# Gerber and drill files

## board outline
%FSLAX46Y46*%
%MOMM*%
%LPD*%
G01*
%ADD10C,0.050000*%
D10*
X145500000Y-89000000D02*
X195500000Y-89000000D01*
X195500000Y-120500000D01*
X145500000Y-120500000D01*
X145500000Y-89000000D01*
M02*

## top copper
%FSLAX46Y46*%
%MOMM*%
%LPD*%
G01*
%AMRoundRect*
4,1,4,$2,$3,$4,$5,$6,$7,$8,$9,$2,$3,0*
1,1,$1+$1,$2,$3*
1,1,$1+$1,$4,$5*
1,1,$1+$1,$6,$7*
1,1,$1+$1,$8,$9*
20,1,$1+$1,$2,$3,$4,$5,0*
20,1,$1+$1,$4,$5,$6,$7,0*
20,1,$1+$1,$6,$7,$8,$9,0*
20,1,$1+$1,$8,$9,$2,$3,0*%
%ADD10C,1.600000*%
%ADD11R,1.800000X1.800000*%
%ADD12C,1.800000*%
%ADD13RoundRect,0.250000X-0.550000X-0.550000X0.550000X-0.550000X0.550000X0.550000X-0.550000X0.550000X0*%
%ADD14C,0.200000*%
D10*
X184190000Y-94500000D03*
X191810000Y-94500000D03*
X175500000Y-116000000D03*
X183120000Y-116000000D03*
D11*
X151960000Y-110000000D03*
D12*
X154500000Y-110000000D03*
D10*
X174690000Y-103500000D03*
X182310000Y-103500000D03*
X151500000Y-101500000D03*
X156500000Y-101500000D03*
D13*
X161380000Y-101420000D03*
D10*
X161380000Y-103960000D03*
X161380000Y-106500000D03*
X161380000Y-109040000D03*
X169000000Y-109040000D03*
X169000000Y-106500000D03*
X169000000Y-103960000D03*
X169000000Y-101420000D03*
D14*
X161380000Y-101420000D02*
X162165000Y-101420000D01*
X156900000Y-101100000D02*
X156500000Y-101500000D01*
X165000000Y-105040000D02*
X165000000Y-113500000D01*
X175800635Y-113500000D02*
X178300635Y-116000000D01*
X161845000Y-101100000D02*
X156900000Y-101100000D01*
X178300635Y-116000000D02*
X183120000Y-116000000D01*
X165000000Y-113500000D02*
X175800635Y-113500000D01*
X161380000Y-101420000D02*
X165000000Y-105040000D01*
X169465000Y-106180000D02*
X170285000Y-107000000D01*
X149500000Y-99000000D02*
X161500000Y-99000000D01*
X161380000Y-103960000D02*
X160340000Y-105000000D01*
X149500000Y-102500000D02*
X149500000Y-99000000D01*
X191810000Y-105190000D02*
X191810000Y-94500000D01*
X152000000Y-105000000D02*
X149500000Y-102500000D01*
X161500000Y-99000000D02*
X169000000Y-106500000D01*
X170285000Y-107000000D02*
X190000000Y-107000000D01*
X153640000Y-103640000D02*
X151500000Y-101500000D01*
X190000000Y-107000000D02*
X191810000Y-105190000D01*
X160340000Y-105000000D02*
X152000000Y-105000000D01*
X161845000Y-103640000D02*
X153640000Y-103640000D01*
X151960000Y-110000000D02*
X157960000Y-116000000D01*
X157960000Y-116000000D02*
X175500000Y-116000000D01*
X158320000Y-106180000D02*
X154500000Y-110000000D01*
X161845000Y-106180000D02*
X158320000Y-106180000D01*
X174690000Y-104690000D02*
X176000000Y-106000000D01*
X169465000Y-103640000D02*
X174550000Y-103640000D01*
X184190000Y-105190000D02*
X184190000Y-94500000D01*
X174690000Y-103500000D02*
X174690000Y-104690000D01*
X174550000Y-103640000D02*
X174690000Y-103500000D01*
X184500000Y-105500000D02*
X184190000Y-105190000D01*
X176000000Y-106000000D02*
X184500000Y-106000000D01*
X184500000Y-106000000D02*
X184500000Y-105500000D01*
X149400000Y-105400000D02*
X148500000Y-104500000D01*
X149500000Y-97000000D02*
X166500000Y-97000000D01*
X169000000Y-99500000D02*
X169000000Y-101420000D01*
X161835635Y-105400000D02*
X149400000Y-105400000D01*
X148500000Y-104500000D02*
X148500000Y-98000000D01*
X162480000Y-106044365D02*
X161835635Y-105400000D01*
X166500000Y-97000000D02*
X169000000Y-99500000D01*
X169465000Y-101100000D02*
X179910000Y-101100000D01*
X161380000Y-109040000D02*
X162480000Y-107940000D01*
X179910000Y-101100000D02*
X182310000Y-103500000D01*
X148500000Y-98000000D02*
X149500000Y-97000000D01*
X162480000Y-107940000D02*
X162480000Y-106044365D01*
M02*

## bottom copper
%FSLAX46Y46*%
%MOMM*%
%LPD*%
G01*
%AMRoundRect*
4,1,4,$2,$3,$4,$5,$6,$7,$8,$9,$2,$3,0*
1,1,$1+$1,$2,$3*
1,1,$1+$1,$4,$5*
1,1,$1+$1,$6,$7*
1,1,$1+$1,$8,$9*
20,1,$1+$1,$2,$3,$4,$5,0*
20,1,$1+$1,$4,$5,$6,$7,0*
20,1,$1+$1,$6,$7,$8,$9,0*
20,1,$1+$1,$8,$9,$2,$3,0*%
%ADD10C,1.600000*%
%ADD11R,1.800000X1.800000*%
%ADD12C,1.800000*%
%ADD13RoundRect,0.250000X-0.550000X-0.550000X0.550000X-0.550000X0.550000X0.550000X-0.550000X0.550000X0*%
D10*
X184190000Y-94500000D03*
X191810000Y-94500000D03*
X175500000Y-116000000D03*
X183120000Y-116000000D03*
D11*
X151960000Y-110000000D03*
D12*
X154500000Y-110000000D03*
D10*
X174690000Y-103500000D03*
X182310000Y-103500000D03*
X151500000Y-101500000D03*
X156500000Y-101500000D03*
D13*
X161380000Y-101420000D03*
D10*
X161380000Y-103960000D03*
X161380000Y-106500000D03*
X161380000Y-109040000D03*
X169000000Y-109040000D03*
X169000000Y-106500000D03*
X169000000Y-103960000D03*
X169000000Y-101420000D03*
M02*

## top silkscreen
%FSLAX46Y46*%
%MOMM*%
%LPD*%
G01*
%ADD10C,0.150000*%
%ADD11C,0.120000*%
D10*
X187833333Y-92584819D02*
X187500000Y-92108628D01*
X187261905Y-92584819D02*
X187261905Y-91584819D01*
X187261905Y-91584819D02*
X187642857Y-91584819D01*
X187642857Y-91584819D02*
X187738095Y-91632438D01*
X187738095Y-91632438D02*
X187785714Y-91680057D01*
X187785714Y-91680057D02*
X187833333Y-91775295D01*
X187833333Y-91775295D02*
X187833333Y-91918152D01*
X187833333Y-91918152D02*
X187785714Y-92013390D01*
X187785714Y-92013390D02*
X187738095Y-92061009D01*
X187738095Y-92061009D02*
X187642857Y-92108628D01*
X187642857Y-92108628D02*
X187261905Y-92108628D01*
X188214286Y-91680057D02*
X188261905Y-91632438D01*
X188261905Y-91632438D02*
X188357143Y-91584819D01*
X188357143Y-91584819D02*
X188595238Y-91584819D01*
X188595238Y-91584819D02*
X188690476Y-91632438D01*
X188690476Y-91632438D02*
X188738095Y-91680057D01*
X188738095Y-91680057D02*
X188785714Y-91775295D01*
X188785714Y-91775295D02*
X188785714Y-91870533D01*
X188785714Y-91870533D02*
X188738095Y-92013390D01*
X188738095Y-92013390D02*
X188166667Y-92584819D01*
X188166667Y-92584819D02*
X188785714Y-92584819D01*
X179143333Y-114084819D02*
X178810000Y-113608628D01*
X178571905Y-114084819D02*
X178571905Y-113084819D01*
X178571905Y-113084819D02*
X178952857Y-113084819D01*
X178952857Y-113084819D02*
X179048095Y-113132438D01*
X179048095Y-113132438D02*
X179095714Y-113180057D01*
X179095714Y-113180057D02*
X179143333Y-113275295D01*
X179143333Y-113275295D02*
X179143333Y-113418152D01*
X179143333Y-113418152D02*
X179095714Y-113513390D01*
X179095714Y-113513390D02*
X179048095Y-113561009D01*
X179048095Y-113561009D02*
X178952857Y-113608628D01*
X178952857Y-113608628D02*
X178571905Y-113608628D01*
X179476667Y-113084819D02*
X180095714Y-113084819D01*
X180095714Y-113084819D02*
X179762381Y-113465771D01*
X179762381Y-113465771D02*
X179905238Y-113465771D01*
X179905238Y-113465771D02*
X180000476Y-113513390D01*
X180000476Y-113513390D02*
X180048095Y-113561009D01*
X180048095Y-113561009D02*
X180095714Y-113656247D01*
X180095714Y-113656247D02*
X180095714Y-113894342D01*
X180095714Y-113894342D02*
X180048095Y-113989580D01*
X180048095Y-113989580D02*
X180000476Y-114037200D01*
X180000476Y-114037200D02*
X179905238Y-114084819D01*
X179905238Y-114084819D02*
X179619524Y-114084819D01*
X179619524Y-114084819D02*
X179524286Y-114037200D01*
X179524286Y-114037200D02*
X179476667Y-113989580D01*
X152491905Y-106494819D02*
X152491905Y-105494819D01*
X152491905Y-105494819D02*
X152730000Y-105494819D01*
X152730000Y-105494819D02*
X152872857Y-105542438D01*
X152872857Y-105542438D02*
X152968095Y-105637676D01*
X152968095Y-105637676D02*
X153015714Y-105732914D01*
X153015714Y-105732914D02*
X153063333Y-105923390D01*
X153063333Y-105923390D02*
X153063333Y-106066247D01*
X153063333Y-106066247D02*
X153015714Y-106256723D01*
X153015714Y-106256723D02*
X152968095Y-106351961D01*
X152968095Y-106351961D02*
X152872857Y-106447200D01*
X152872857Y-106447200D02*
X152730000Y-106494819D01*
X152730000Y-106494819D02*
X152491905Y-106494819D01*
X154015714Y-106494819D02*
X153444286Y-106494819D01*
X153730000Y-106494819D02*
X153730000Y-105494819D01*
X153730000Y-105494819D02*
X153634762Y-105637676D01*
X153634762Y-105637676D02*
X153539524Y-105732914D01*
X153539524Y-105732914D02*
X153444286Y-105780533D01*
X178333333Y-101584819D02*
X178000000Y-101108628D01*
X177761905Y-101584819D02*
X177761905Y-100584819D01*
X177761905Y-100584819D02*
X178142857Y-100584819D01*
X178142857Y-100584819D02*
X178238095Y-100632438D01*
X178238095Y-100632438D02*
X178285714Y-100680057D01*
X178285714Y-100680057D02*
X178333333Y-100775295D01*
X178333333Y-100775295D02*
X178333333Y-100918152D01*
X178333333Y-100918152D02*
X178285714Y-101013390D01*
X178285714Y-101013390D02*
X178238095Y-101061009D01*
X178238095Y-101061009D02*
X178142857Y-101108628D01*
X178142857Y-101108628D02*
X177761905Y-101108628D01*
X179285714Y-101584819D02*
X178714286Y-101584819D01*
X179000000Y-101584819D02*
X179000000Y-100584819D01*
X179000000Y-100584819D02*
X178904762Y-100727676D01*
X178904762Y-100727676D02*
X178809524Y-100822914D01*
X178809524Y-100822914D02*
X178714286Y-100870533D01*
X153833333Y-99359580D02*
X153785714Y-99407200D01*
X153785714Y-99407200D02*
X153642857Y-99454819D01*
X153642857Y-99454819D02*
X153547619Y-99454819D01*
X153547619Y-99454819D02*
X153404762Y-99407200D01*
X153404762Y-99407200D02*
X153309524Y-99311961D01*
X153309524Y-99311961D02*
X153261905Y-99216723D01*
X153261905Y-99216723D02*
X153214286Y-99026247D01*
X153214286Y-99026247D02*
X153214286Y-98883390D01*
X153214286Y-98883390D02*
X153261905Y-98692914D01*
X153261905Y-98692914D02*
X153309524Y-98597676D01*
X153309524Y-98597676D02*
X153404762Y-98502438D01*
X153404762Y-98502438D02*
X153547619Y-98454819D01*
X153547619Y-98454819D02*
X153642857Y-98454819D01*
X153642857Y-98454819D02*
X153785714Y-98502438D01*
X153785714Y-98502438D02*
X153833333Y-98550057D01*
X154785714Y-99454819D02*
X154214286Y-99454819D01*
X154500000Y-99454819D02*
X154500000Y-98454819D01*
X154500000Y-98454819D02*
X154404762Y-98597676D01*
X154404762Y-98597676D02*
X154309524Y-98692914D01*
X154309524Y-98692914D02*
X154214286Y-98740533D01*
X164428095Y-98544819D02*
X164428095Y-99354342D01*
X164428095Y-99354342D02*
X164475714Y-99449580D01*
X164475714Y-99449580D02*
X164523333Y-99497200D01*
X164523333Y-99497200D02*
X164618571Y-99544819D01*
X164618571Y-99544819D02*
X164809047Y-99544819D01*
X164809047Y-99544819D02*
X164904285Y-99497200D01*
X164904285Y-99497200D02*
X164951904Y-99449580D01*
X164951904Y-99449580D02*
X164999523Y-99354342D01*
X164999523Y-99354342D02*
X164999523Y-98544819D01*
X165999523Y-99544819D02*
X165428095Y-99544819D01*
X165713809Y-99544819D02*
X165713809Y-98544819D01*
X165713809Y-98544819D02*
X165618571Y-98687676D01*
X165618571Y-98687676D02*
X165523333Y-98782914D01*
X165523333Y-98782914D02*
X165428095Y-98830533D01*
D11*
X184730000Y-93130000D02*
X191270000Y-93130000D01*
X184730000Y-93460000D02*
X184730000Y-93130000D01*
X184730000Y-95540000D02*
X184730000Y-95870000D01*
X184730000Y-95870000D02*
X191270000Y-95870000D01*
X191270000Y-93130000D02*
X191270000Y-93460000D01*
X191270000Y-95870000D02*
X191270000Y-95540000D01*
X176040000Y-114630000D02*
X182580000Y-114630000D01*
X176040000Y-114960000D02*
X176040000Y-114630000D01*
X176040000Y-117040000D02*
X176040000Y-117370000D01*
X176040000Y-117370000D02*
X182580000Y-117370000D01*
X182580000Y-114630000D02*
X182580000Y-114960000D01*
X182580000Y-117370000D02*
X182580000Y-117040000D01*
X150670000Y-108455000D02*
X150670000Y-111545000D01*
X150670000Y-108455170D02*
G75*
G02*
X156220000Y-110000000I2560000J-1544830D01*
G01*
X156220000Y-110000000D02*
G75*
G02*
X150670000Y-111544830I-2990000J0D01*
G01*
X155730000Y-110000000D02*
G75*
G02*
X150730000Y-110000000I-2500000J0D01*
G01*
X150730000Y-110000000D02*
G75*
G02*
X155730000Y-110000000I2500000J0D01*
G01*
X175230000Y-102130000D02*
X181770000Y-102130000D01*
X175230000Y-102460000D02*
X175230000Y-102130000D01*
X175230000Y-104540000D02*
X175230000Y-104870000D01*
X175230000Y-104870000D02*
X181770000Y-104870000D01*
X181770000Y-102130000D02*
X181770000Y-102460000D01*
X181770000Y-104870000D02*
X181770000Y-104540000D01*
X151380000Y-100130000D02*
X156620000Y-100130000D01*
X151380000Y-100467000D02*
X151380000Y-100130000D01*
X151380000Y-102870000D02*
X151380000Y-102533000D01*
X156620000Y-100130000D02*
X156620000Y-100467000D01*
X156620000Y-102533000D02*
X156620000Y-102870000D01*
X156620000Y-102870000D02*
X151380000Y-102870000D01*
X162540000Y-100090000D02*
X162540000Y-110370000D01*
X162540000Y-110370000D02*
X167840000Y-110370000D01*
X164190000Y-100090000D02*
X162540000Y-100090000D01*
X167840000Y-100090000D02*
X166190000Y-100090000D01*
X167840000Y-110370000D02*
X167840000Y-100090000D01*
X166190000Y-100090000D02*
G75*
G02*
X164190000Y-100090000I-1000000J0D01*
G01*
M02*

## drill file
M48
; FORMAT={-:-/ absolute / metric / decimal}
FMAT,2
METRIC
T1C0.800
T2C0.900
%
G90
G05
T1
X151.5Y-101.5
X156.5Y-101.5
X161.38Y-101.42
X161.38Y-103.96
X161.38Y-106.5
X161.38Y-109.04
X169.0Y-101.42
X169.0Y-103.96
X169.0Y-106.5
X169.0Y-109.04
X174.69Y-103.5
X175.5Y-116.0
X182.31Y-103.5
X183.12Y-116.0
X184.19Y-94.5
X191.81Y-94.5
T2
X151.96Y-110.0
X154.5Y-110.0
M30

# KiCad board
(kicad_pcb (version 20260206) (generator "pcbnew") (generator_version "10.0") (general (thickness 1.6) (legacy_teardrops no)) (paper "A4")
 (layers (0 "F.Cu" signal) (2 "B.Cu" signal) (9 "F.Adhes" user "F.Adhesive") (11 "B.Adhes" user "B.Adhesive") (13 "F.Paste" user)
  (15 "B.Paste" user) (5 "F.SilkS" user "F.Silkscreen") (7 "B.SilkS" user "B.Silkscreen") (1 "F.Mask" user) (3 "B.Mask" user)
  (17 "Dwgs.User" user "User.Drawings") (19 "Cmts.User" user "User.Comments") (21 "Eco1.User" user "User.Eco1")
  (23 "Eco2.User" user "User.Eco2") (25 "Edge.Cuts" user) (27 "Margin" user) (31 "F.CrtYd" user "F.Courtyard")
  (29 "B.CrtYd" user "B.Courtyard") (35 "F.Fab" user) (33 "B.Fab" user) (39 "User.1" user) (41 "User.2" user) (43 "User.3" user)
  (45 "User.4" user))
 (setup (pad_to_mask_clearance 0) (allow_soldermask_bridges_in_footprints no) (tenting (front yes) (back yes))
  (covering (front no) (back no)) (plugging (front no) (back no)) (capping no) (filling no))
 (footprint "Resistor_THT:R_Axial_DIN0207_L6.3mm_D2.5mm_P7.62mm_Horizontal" (layer "F.Cu") (at 184.19 94.5)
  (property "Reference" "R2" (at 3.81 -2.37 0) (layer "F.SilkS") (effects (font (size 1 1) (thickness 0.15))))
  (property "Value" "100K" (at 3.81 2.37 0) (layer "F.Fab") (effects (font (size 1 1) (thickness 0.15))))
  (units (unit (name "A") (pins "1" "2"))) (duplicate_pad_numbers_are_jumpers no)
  (fp_line (start 0.54 -1.37) (end 7.08 -1.37) (stroke (width 0.12) (type solid)) (layer "F.SilkS"))
  (fp_line (start 0.54 -1.04) (end 0.54 -1.37) (stroke (width 0.12) (type solid)) (layer "F.SilkS"))
  (fp_line (start 0.54 1.04) (end 0.54 1.37) (stroke (width 0.12) (type solid)) (layer "F.SilkS"))
  (fp_line (start 0.54 1.37) (end 7.08 1.37) (stroke (width 0.12) (type solid)) (layer "F.SilkS"))
  (fp_line (start 7.08 -1.37) (end 7.08 -1.04) (stroke (width 0.12) (type solid)) (layer "F.SilkS"))
  (fp_line (start 7.08 1.37) (end 7.08 1.04) (stroke (width 0.12) (type solid)) (layer "F.SilkS"))
  (pad "1" thru_hole circle (at 0 0) (size 1.6 1.6) (drill 0.8) (layers "*.Cu" "*.Mask") (remove_unused_layers no) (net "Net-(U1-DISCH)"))
  (pad "2" thru_hole circle (at 7.62 0) (size 1.6 1.6) (drill 0.8) (layers "*.Cu" "*.Mask") (remove_unused_layers no) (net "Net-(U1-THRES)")))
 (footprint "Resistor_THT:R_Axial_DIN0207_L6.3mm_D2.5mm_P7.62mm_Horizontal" (layer "F.Cu") (at 175.5 116)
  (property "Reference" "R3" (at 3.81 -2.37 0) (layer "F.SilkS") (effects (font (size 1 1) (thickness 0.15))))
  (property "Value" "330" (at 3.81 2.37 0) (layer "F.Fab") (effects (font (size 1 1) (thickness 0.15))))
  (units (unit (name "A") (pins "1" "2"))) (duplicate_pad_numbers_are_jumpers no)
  (fp_line (start 0.54 -1.37) (end 7.08 -1.37) (stroke (width 0.12) (type solid)) (layer "F.SilkS"))
  (fp_line (start 0.54 -1.04) (end 0.54 -1.37) (stroke (width 0.12) (type solid)) (layer "F.SilkS"))
  (fp_line (start 0.54 1.04) (end 0.54 1.37) (stroke (width 0.12) (type solid)) (layer "F.SilkS"))
  (fp_line (start 0.54 1.37) (end 7.08 1.37) (stroke (width 0.12) (type solid)) (layer "F.SilkS"))
  (fp_line (start 7.08 -1.37) (end 7.08 -1.04) (stroke (width 0.12) (type solid)) (layer "F.SilkS"))
  (fp_line (start 7.08 1.37) (end 7.08 1.04) (stroke (width 0.12) (type solid)) (layer "F.SilkS"))
  (pad "1" thru_hole circle (at 0 0) (size 1.6 1.6) (drill 0.8) (layers "*.Cu" "*.Mask") (remove_unused_layers no) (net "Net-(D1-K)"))
  (pad "2" thru_hole circle (at 7.62 0) (size 1.6 1.6) (drill 0.8) (layers "*.Cu" "*.Mask") (remove_unused_layers no) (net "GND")))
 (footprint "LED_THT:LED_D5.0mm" (layer "F.Cu") (at 151.96 110)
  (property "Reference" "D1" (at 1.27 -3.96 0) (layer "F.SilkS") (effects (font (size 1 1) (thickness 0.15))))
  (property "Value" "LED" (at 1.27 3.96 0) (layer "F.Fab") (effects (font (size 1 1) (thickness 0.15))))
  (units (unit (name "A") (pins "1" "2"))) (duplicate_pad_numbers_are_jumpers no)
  (fp_line (start -1.29 -1.545) (end -1.29 1.545) (stroke (width 0.12) (type solid)) (layer "F.SilkS"))
  (fp_arc (start -1.29 -1.54483) (mid 2.071779 -2.880495) (end 4.26 0) (stroke (width 0.12) (type solid)) (layer "F.SilkS"))
  (fp_arc (start 4.26 0) (mid 2.071779 2.880495) (end -1.29 1.54483) (stroke (width 0.12) (type solid)) (layer "F.SilkS"))
  (fp_circle (center 1.27 0) (end 3.77 0) (stroke (width 0.12) (type solid)) (fill no) (layer "F.SilkS"))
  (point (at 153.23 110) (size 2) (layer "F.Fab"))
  (pad "1" thru_hole rect (at 0 0) (size 1.8 1.8) (drill 0.9) (layers "*.Cu" "*.Mask") (remove_unused_layers no) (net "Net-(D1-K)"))
  (pad "2" thru_hole circle (at 2.54 0) (size 1.8 1.8) (drill 0.9) (layers "*.Cu" "*.Mask") (remove_unused_layers no) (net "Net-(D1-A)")))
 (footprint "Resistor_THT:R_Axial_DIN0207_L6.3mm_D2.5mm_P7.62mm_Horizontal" (layer "F.Cu") (at 174.69 103.5)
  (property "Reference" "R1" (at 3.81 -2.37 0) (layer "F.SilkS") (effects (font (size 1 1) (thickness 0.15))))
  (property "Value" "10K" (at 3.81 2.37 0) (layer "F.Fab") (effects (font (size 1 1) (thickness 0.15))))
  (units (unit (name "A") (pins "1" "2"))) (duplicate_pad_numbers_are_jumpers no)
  (fp_line (start 0.54 -1.37) (end 7.08 -1.37) (stroke (width 0.12) (type solid)) (layer "F.SilkS"))
  (fp_line (start 0.54 -1.04) (end 0.54 -1.37) (stroke (width 0.12) (type solid)) (layer "F.SilkS"))
  (fp_line (start 0.54 1.04) (end 0.54 1.37) (stroke (width 0.12) (type solid)) (layer "F.SilkS"))
  (fp_line (start 0.54 1.37) (end 7.08 1.37) (stroke (width 0.12) (type solid)) (layer "F.SilkS"))
  (fp_line (start 7.08 -1.37) (end 7.08 -1.04) (stroke (width 0.12) (type solid)) (layer "F.SilkS"))
  (fp_line (start 7.08 1.37) (end 7.08 1.04) (stroke (width 0.12) (type solid)) (layer "F.SilkS"))
  (pad "1" thru_hole circle (at 0 0) (size 1.6 1.6) (drill 0.8) (layers "*.Cu" "*.Mask") (remove_unused_layers no) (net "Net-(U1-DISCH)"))
  (pad "2" thru_hole circle (at 7.62 0) (size 1.6 1.6) (drill 0.8) (layers "*.Cu" "*.Mask") (remove_unused_layers no) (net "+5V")))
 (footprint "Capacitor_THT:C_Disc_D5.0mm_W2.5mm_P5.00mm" (layer "F.Cu") (at 151.5 101.5)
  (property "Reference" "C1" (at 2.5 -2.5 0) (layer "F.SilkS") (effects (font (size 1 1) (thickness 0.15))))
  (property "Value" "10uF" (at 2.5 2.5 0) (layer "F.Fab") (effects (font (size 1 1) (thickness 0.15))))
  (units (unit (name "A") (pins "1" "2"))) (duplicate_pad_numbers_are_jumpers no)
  (fp_line (start -0.12 -1.37) (end 5.12 -1.37) (stroke (width 0.12) (type solid)) (layer "F.SilkS"))
  (fp_line (start -0.12 -1.033) (end -0.12 -1.37) (stroke (width 0.12) (type solid)) (layer "F.SilkS"))
  (fp_line (start -0.12 1.37) (end -0.12 1.033) (stroke (width 0.12) (type solid)) (layer "F.SilkS"))
  (fp_line (start 5.12 -1.37) (end 5.12 -1.033) (stroke (width 0.12) (type solid)) (layer "F.SilkS"))
  (fp_line (start 5.12 1.033) (end 5.12 1.37) (stroke (width 0.12) (type solid)) (layer "F.SilkS"))
  (fp_line (start 5.12 1.37) (end -0.12 1.37) (stroke (width 0.12) (type solid)) (layer "F.SilkS"))
  (pad "1" thru_hole circle (at 0 0) (size 1.6 1.6) (drill 0.8) (layers "*.Cu" "*.Mask") (remove_unused_layers no) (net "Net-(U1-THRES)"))
  (pad "2" thru_hole circle (at 5 0) (size 1.6 1.6) (drill 0.8) (layers "*.Cu" "*.Mask") (remove_unused_layers no) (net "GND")))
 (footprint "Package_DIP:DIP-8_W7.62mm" (layer "F.Cu") (at 161.38 101.42)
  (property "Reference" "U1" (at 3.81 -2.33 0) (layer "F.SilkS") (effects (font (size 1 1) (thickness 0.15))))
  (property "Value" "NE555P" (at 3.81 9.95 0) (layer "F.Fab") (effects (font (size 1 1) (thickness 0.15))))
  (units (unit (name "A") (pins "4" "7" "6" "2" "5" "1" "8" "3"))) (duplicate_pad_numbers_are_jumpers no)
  (fp_line (start 1.16 -1.33) (end 1.16 8.95) (stroke (width 0.12) (type solid)) (layer "F.SilkS"))
  (fp_line (start 1.16 8.95) (end 6.46 8.95) (stroke (width 0.12) (type solid)) (layer "F.SilkS"))
  (fp_line (start 2.81 -1.33) (end 1.16 -1.33) (stroke (width 0.12) (type solid)) (layer "F.SilkS"))
  (fp_line (start 6.46 -1.33) (end 4.81 -1.33) (stroke (width 0.12) (type solid)) (layer "F.SilkS"))
  (fp_line (start 6.46 8.95) (end 6.46 -1.33) (stroke (width 0.12) (type solid)) (layer "F.SilkS"))
  (fp_arc (start 4.81 -1.33) (mid 3.81 -0.33) (end 2.81 -1.33) (stroke (width 0.12) (type solid)) (layer "F.SilkS"))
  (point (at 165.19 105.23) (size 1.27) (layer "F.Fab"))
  (pad "1" thru_hole roundrect (at 0 0) (size 1.6 1.6) (drill 0.8) (layers "*.Cu" "*.Mask") (remove_unused_layers no)
   (roundrect_rratio 0.15625) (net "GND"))
  (pad "2" thru_hole circle (at 0 2.54) (size 1.6 1.6) (drill 0.8) (layers "*.Cu" "*.Mask") (remove_unused_layers no) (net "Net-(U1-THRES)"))
  (pad "3" thru_hole circle (at 0 5.08) (size 1.6 1.6) (drill 0.8) (layers "*.Cu" "*.Mask") (remove_unused_layers no) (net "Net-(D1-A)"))
  (pad "4" thru_hole circle (at 0 7.62) (size 1.6 1.6) (drill 0.8) (layers "*.Cu" "*.Mask") (remove_unused_layers no) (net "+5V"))
  (pad "5" thru_hole circle (at 7.62 7.62) (size 1.6 1.6) (drill 0.8) (layers "*.Cu" "*.Mask") (remove_unused_layers no)
   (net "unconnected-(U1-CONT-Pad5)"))
  (pad "6" thru_hole circle (at 7.62 5.08) (size 1.6 1.6) (drill 0.8) (layers "*.Cu" "*.Mask") (remove_unused_layers no)
   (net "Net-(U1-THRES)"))
  (pad "7" thru_hole circle (at 7.62 2.54) (size 1.6 1.6) (drill 0.8) (layers "*.Cu" "*.Mask") (remove_unused_layers no)
   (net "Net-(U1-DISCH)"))
  (pad "8" thru_hole circle (at 7.62 0) (size 1.6 1.6) (drill 0.8) (layers "*.Cu" "*.Mask") (remove_unused_layers no) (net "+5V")))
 (gr_rect (start 145.5 89) (end 195.5 120.5) (stroke (width 0.05) (type default)) (fill no) (layer "Edge.Cuts"))
 (segment (start 161.38 101.42) (end 162.165 101.42) (width 0.2) (layer "F.Cu") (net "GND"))
 (segment (start 156.9 101.1) (end 156.5 101.5) (width 0.2) (layer "F.Cu") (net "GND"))
 (segment (start 165 105.04) (end 165 113.5) (width 0.2) (layer "F.Cu") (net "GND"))
 (segment (start 175.800635 113.5) (end 178.300635 116) (width 0.2) (layer "F.Cu") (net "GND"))
 (segment (start 161.845 101.1) (end 156.9 101.1) (width 0.2) (layer "F.Cu") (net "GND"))
 (segment (start 178.300635 116) (end 183.12 116) (width 0.2) (layer "F.Cu") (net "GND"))
 (segment (start 165 113.5) (end 175.800635 113.5) (width 0.2) (layer "F.Cu") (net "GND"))
 (segment (start 161.38 101.42) (end 165 105.04) (width 0.2) (layer "F.Cu") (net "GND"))
 (segment (start 169.465 106.18) (end 170.285 107) (width 0.2) (layer "F.Cu") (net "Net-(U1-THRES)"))
 (segment (start 149.5 99) (end 161.5 99) (width 0.2) (layer "F.Cu") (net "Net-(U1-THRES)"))
 (segment (start 161.38 103.96) (end 160.34 105) (width 0.2) (layer "F.Cu") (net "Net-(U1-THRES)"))
 (segment (start 149.5 102.5) (end 149.5 99) (width 0.2) (layer "F.Cu") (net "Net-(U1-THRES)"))
 (segment (start 191.81 105.19) (end 191.81 94.5) (width 0.2) (layer "F.Cu") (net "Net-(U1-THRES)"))
 (segment (start 152 105) (end 149.5 102.5) (width 0.2) (layer "F.Cu") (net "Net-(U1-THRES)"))
 (segment (start 161.5 99) (end 169 106.5) (width 0.2) (layer "F.Cu") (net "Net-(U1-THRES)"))
 (segment (start 170.285 107) (end 190 107) (width 0.2) (layer "F.Cu") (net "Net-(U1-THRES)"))
 (segment (start 153.64 103.64) (end 151.5 101.5) (width 0.2) (layer "F.Cu") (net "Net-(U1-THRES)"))
 (segment (start 190 107) (end 191.81 105.19) (width 0.2) (layer "F.Cu") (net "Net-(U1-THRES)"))
 (segment (start 160.34 105) (end 152 105) (width 0.2) (layer "F.Cu") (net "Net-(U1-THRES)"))
 (segment (start 161.845 103.64) (end 153.64 103.64) (width 0.2) (layer "F.Cu") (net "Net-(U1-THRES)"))
 (segment (start 151.96 110) (end 157.96 116) (width 0.2) (layer "F.Cu") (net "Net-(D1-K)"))
 (segment (start 157.96 116) (end 175.5 116) (width 0.2) (layer "F.Cu") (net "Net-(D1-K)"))
 (segment (start 158.32 106.18) (end 154.5 110) (width 0.2) (layer "F.Cu") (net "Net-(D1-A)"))
 (segment (start 161.845 106.18) (end 158.32 106.18) (width 0.2) (layer "F.Cu") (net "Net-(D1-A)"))
 (segment (start 174.69 104.69) (end 176 106) (width 0.2) (layer "F.Cu") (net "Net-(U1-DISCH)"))
 (segment (start 169.465 103.64) (end 174.55 103.64) (width 0.2) (layer "F.Cu") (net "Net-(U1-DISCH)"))
 (segment (start 184.19 105.19) (end 184.19 94.5) (width 0.2) (layer "F.Cu") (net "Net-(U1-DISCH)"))
 (segment (start 174.69 103.5) (end 174.69 104.69) (width 0.2) (layer "F.Cu") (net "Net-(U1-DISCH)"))
 (segment (start 174.55 103.64) (end 174.69 103.5) (width 0.2) (layer "F.Cu") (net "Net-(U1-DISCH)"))
 (segment (start 184.5 105.5) (end 184.19 105.19) (width 0.2) (layer "F.Cu") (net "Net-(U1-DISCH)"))
 (segment (start 176 106) (end 184.5 106) (width 0.2) (layer "F.Cu") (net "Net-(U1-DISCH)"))
 (segment (start 184.5 106) (end 184.5 105.5) (width 0.2) (layer "F.Cu") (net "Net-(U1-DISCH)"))
 (segment (start 149.4 105.4) (end 148.5 104.5) (width 0.2) (layer "F.Cu") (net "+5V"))
 (segment (start 149.5 97) (end 166.5 97) (width 0.2) (layer "F.Cu") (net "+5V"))
 (segment (start 169 99.5) (end 169 101.42) (width 0.2) (layer "F.Cu") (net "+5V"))
 (segment (start 161.835635 105.4) (end 149.4 105.4) (width 0.2) (layer "F.Cu") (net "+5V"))
 (segment (start 148.5 104.5) (end 148.5 98) (width 0.2) (layer "F.Cu") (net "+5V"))
 (segment (start 162.48 106.044365) (end 161.835635 105.4) (width 0.2) (layer "F.Cu") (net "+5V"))
 (segment (start 166.5 97) (end 169 99.5) (width 0.2) (layer "F.Cu") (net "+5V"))
 (segment (start 169.465 101.1) (end 179.91 101.1) (width 0.2) (layer "F.Cu") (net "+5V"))
 (segment (start 161.38 109.04) (end 162.48 107.94) (width 0.2) (layer "F.Cu") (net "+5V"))
 (segment (start 179.91 101.1) (end 182.31 103.5) (width 0.2) (layer "F.Cu") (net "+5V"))
 (segment (start 148.5 98) (end 149.5 97) (width 0.2) (layer "F.Cu") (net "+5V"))
 (segment (start 162.48 107.94) (end 162.48 106.044365) (width 0.2) (layer "F.Cu") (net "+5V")))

